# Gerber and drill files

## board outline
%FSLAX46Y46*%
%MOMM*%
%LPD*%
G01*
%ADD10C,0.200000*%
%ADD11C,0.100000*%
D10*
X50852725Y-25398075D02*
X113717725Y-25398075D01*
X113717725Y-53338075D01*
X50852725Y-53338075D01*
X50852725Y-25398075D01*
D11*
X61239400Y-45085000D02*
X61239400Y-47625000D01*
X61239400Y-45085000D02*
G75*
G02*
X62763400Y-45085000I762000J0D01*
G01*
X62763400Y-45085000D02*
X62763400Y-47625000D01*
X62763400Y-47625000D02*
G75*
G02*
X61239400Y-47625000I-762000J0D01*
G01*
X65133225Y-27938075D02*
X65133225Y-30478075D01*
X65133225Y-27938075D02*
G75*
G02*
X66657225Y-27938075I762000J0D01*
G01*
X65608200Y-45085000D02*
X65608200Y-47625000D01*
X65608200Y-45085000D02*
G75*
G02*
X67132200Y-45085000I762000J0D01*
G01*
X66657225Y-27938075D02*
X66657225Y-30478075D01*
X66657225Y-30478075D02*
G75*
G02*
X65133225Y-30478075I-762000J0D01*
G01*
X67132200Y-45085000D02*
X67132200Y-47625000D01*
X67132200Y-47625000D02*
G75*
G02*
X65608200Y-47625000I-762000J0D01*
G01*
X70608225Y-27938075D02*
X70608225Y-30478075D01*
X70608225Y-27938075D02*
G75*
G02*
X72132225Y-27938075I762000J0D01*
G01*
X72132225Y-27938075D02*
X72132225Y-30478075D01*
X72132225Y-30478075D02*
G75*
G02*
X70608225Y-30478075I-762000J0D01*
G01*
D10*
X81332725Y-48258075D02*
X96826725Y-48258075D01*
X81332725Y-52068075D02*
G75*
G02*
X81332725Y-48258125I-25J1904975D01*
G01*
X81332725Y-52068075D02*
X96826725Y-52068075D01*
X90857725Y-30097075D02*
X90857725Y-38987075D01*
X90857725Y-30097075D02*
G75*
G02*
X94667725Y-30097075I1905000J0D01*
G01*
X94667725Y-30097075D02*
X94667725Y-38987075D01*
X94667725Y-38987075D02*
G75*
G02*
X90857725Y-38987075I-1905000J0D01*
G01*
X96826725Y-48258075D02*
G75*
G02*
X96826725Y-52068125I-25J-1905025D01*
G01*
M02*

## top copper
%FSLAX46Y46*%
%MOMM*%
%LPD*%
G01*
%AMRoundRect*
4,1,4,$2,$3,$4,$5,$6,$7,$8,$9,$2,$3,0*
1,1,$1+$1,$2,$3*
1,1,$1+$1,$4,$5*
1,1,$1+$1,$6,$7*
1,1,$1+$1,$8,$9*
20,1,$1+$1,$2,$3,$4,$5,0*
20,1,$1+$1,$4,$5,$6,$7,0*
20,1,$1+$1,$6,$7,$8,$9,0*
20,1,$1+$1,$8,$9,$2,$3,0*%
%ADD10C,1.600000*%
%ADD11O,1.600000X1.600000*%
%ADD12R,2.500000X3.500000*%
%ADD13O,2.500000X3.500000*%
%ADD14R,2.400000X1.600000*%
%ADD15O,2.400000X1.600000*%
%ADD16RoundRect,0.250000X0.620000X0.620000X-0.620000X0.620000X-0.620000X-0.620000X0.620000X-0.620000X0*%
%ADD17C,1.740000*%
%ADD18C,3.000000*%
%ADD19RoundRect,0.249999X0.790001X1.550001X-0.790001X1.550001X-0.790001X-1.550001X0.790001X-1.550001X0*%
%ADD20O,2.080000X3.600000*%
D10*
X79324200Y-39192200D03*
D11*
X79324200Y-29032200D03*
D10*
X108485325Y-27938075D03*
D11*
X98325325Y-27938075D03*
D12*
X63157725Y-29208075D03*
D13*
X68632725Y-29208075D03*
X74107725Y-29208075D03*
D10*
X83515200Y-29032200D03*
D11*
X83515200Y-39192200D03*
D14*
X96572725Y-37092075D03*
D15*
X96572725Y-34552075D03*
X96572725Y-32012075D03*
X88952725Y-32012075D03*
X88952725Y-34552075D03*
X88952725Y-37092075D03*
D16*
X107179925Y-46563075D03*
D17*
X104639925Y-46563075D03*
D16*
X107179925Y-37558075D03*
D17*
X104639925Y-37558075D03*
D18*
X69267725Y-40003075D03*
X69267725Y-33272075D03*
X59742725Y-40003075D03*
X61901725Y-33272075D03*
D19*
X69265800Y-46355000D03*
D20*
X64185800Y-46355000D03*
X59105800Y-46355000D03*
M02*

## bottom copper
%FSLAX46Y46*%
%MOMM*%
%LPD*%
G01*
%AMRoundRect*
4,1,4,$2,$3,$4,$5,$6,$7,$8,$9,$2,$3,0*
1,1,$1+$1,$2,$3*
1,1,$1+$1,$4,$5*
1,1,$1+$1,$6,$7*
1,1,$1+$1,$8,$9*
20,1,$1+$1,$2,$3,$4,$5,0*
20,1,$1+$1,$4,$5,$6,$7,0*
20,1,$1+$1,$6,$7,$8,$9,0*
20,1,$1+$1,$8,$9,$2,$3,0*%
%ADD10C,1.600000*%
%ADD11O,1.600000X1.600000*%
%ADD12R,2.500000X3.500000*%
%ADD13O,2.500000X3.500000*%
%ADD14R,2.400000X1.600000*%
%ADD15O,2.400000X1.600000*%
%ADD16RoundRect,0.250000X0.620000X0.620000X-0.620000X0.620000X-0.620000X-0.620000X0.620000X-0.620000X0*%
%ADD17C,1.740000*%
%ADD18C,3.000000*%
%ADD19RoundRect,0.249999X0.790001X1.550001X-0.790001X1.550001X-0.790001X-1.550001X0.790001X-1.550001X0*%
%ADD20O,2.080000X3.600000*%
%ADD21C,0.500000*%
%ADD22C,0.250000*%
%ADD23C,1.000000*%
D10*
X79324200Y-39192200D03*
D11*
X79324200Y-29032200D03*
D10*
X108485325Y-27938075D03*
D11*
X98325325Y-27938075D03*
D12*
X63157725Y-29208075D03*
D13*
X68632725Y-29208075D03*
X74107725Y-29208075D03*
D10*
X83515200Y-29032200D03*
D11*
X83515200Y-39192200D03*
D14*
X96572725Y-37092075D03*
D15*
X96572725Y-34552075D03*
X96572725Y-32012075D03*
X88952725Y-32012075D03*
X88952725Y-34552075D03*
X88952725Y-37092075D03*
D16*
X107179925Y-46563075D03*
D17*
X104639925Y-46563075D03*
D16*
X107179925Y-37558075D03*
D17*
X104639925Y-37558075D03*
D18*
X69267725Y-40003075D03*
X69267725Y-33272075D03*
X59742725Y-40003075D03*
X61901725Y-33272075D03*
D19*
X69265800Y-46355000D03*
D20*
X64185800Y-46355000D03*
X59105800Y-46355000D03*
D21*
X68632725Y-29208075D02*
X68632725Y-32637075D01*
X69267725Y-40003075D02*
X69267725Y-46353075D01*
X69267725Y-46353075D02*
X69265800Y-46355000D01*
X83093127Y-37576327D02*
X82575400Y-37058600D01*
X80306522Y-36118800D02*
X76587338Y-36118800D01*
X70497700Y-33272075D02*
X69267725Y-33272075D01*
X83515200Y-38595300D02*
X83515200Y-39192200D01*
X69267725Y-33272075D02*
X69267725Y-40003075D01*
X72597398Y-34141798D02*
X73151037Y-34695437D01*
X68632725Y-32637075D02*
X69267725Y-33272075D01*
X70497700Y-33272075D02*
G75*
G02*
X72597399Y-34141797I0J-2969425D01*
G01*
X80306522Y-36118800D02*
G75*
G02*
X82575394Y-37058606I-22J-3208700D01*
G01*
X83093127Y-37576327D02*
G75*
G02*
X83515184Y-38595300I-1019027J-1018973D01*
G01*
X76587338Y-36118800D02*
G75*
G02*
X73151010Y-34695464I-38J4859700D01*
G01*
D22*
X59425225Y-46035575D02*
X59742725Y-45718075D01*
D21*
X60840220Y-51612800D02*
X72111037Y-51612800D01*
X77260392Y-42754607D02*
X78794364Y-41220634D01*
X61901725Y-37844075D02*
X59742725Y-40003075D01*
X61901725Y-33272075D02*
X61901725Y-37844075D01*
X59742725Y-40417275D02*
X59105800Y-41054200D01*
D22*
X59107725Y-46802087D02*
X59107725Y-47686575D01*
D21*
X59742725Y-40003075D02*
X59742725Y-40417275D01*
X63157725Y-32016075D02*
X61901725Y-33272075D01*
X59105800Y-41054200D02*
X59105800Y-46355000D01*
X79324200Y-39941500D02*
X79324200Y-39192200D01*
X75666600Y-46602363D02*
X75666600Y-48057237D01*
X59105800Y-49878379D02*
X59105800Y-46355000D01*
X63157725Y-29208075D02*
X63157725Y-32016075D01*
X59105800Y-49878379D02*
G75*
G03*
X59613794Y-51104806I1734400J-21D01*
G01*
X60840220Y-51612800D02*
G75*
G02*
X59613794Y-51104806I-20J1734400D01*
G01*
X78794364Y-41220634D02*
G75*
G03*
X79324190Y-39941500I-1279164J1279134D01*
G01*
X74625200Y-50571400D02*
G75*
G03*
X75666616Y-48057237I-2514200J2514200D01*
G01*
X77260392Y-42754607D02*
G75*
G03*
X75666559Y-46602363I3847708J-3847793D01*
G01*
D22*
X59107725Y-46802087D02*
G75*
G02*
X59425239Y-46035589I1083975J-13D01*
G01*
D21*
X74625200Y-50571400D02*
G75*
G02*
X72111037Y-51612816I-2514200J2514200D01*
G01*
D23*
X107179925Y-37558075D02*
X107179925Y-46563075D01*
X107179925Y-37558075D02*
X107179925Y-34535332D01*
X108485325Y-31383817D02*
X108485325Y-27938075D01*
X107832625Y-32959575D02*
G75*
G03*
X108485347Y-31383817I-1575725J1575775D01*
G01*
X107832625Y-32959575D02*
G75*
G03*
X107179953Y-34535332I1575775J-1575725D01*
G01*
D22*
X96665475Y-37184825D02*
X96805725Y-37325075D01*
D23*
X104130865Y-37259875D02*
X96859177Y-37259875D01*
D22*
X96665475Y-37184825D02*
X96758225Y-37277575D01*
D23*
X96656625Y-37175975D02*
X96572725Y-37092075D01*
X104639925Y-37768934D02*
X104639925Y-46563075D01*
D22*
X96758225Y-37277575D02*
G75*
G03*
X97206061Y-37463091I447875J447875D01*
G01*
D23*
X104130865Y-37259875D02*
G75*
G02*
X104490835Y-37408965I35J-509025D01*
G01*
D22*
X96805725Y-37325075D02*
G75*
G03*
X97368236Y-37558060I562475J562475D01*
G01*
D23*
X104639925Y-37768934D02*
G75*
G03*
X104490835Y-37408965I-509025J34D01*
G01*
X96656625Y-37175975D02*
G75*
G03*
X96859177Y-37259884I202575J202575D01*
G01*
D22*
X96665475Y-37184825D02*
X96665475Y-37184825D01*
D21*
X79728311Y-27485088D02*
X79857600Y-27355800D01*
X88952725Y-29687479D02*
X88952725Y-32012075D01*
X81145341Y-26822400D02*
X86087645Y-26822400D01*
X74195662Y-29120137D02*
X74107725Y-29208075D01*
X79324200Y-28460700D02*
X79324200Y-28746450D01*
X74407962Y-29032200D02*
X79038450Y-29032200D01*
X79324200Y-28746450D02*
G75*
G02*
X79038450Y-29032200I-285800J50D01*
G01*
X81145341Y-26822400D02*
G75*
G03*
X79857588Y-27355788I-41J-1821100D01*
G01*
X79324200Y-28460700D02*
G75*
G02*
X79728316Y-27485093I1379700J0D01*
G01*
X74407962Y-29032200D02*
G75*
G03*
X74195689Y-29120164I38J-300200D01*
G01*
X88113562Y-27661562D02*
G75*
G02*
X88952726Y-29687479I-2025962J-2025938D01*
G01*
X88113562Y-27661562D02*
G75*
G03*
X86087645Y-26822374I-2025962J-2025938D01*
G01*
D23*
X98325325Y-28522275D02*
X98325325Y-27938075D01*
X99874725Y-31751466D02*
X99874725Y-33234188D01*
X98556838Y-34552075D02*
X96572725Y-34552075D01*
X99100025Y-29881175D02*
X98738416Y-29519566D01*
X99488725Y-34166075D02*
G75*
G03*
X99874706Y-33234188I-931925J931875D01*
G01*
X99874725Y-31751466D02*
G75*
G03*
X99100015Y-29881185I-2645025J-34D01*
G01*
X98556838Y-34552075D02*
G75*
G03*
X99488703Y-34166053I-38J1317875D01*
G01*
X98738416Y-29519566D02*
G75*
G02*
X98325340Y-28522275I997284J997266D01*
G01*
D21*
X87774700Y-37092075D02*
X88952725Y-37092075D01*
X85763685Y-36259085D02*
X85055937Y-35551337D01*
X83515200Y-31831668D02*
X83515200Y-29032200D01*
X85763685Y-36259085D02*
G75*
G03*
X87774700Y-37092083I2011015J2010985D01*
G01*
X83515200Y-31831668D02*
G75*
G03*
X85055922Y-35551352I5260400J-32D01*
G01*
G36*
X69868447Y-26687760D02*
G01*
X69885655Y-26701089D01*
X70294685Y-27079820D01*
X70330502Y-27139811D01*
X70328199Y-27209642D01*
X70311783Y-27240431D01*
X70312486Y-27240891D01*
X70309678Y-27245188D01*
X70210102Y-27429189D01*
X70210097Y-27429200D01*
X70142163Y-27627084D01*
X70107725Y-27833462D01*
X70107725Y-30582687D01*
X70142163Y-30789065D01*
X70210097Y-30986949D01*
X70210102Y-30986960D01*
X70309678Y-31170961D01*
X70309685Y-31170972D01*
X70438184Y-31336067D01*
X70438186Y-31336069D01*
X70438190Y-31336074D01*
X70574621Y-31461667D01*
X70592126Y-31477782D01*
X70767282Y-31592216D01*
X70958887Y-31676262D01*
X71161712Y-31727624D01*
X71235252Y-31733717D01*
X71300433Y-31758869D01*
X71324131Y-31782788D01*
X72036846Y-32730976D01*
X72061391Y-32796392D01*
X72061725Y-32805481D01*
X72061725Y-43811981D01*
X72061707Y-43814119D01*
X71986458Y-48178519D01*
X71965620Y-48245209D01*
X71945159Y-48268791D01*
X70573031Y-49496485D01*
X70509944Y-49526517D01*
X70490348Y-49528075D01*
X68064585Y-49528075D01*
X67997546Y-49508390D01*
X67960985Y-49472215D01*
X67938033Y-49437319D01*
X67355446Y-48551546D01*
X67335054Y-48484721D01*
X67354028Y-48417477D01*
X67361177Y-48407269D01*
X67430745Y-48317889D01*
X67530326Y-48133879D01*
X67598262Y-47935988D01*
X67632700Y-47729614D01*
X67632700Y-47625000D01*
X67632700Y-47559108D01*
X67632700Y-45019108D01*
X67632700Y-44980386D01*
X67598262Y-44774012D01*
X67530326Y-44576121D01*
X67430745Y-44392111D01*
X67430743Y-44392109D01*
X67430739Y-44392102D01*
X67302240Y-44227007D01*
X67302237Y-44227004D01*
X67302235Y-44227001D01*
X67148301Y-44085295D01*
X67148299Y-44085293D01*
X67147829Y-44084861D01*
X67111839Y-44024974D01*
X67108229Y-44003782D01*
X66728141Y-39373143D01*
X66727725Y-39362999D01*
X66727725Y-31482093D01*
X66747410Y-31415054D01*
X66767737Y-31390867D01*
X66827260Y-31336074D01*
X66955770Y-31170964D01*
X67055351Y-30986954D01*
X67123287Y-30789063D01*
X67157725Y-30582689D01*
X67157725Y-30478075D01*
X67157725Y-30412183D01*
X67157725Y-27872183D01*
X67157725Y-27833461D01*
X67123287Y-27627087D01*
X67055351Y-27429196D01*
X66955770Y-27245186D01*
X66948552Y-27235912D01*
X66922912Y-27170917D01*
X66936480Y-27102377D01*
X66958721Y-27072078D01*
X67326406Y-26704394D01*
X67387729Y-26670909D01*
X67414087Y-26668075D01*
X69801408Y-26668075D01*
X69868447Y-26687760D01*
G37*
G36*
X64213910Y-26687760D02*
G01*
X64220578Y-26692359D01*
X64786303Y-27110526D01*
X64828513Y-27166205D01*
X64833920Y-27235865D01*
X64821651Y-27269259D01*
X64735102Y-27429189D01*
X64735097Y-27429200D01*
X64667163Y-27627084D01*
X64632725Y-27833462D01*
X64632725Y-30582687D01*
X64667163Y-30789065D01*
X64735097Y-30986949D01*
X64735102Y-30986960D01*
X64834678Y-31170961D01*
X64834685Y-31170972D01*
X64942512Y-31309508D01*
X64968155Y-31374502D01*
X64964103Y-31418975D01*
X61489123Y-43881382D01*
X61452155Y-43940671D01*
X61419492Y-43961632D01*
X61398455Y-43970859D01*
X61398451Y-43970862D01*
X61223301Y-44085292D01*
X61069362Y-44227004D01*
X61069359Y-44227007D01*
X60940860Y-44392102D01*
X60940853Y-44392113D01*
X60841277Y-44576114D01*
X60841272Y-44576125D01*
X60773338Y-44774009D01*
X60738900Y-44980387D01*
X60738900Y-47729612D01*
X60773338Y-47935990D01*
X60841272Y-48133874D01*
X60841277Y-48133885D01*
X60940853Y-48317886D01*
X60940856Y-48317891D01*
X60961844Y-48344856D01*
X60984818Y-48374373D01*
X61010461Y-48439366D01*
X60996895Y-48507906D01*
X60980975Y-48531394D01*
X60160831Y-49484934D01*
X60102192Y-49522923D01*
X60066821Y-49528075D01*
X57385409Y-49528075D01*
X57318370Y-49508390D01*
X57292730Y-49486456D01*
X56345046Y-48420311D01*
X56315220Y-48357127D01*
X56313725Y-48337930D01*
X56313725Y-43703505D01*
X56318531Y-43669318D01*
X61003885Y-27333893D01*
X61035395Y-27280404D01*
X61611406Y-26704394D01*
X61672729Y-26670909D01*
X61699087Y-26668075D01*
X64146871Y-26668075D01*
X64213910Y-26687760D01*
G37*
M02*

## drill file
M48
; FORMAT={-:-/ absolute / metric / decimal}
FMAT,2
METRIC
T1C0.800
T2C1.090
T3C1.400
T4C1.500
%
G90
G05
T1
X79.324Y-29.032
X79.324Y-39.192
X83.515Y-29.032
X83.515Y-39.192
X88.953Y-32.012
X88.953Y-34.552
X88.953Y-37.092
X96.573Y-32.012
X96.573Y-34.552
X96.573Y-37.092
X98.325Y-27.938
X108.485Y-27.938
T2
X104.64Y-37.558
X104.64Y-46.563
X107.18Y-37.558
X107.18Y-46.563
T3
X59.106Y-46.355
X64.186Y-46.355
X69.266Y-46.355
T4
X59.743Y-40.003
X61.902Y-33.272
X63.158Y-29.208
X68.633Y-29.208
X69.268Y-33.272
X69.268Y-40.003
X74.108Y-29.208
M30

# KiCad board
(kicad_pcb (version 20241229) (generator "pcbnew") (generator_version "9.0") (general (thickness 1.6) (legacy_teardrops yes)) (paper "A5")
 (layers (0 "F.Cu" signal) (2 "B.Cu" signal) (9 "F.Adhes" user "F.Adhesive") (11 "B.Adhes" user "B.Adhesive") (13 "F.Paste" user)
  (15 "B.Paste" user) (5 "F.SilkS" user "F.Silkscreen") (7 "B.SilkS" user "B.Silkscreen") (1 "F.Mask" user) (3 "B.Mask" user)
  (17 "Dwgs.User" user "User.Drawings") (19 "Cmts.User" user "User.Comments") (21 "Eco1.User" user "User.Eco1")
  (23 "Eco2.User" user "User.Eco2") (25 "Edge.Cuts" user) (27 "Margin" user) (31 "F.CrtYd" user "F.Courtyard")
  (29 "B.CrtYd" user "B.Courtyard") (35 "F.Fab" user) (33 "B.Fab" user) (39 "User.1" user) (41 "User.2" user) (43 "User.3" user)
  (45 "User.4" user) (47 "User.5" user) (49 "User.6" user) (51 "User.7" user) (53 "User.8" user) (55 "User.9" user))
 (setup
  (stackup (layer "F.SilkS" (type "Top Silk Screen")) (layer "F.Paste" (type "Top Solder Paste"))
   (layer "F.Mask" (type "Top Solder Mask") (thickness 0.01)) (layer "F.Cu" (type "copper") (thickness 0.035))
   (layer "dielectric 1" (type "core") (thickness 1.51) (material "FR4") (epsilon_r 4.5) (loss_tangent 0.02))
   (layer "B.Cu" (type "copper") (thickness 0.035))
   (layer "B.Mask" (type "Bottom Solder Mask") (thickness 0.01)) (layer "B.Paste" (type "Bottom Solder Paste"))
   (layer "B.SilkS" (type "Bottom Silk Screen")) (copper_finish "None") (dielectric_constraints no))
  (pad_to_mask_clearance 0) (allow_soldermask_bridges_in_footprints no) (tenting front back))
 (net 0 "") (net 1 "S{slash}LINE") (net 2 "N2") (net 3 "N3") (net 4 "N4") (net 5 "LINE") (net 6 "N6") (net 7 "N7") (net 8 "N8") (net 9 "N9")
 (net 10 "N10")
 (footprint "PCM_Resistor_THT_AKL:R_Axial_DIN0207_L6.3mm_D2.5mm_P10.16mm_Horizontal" (layer "F.Cu") (at 79.3242 39.1922 90)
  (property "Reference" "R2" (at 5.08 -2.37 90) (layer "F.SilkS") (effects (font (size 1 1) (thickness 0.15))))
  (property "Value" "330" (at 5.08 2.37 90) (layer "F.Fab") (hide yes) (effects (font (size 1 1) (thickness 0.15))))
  (pad "1" thru_hole circle (at 0 0 90) (size 1.6 1.6) (drill 0.8) (layers "*.Cu" "*.Mask") (remove_unused_layers no) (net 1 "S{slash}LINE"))
  (pad "2" thru_hole oval (at 10.16 0 90) (size 1.6 1.6) (drill 0.8) (layers "*.Cu" "*.Mask") (remove_unused_layers no) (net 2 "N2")))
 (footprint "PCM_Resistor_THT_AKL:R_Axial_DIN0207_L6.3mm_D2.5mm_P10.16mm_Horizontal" (layer "F.Cu") (at 108.485325 27.938075 180)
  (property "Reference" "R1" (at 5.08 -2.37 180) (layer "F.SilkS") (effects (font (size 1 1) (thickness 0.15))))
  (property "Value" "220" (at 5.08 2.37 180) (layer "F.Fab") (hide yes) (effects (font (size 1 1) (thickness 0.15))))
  (pad "1" thru_hole circle (at 0 0 180) (size 1.6 1.6) (drill 0.8) (layers "*.Cu" "*.Mask") (remove_unused_layers no) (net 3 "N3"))
  (pad "2" thru_hole oval (at 10.16 0 180) (size 1.6 1.6) (drill 0.8) (layers "*.Cu" "*.Mask") (remove_unused_layers no) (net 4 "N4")))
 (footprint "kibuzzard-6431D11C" (layer "F.Cu") (at 53.011725 39.368075 90)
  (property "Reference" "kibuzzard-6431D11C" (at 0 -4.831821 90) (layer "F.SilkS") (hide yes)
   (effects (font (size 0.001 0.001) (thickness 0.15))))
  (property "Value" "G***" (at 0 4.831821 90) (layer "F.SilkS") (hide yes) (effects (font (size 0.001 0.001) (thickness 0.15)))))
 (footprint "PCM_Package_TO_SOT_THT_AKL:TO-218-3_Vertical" (layer "F.Cu") (at 63.157725 29.208075)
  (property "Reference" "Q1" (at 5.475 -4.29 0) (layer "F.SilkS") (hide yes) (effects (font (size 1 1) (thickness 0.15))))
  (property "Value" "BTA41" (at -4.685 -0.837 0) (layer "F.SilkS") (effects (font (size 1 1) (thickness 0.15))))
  (pad "1" thru_hole rect (at 0 0) (size 2.5 3.5) (drill 1.5) (layers "*.Cu" "*.Mask") (remove_unused_layers no) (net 1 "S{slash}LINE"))
  (pad "2" thru_hole oval (at 5.475 0) (size 2.5 3.5) (drill 1.5) (layers "*.Cu" "*.Mask") (remove_unused_layers no) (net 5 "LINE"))
  (pad "3" thru_hole oval (at 10.95 0) (size 2.5 3.5) (drill 1.5) (layers "*.Cu" "*.Mask") (remove_unused_layers no) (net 2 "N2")))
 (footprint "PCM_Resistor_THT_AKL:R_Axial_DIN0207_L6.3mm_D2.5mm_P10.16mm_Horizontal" (layer "F.Cu") (at 83.5152 29.0322 -90)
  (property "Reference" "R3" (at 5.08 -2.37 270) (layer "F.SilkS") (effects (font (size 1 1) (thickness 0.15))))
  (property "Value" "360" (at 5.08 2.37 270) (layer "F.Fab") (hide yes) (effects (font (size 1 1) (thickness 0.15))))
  (pad "1" thru_hole circle (at 0 0 270) (size 1.6 1.6) (drill 0.8) (layers "*.Cu" "*.Mask") (remove_unused_layers no) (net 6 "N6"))
  (pad "2" thru_hole oval (at 10.16 0 270) (size 1.6 1.6) (drill 0.8) (layers "*.Cu" "*.Mask") (remove_unused_layers no) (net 5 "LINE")))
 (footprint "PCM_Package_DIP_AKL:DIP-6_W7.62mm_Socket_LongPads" (layer "F.Cu") (at 96.572725 37.092075 180)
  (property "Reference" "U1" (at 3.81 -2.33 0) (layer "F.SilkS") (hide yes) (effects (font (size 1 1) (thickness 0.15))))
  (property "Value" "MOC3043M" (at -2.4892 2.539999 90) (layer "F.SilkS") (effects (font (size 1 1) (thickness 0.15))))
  (pad "1" thru_hole rect (at 0 0 180) (size 2.4 1.6) (drill 0.8) (layers "*.Cu" "*.Mask") (remove_unused_layers no) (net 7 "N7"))
  (pad "2" thru_hole oval (at 0 2.54 180) (size 2.4 1.6) (drill 0.8) (layers "*.Cu" "*.Mask") (remove_unused_layers no) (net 4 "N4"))
  (pad "3" thru_hole oval (at 0 5.08 180) (size 2.4 1.6) (drill 0.8) (layers "*.Cu" "*.Mask") (remove_unused_layers no) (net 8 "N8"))
  (pad "4" thru_hole oval (at 7.62 5.08 180) (size 2.4 1.6) (drill 0.8) (layers "*.Cu" "*.Mask") (remove_unused_layers no) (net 2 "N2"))
  (pad "5" thru_hole oval (at 7.62 2.54 180) (size 2.4 1.6) (drill 0.8) (layers "*.Cu" "*.Mask") (remove_unused_layers no) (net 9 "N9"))
  (pad "6" thru_hole oval (at 7.62 0 180) (size 2.4 1.6) (drill 0.8) (layers "*.Cu" "*.Mask") (remove_unused_layers no) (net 6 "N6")))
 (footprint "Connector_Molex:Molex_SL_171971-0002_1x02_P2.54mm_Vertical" (layer "F.Cu") (at 107.179925 46.563075 180)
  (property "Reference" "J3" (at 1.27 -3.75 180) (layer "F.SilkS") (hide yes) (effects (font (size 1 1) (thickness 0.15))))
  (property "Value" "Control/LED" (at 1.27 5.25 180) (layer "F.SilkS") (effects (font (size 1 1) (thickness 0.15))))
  (pad "1" thru_hole roundrect (at 0 0 180) (size 1.74 1.74) (drill 1.09) (layers "*.Cu" "*.Mask") (remove_unused_layers no)
   (roundrect_rratio 0.143678) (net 3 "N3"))
  (pad "2" thru_hole circle (at 2.54 0 180) (size 1.74 1.74) (drill 1.09) (layers "*.Cu" "*.Mask") (remove_unused_layers no) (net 7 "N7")))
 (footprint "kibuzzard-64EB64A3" (layer "F.Cu") (at 112.041325 39.368075 -90)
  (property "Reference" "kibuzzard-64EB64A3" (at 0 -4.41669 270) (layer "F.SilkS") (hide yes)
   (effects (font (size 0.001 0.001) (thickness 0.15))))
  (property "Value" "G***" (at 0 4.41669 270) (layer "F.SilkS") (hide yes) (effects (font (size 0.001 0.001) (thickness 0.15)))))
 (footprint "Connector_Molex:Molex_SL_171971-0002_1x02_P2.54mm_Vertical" (layer "F.Cu") (at 107.179925 37.558075 180)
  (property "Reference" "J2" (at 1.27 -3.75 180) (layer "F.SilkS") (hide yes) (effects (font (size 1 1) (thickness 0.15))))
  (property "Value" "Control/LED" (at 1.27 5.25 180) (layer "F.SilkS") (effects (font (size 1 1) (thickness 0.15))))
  (pad "1" thru_hole roundrect (at 0 0 180) (size 1.74 1.74) (drill 1.09) (layers "*.Cu" "*.Mask") (remove_unused_layers no)
   (roundrect_rratio 0.143678) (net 3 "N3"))
  (pad "2" thru_hole circle (at 2.54 0 180) (size 1.74 1.74) (drill 1.09) (layers "*.Cu" "*.Mask") (remove_unused_layers no) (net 7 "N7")))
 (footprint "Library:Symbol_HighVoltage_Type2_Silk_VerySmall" (layer "F.Cu") (at 85.549125 44.676675)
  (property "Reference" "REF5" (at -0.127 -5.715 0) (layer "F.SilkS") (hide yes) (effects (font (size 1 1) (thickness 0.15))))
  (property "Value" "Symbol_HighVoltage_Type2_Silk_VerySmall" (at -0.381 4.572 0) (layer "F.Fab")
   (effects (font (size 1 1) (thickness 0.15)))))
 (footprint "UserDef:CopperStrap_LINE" (layer "F.Cu") (at 69.267725 40.003075)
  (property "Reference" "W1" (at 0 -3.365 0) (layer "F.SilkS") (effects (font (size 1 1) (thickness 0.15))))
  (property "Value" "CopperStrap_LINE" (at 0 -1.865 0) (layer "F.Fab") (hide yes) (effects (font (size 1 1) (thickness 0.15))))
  (pad "1" thru_hole circle (at 0 0) (size 3 3) (drill 1.5) (layers "*.Cu" "*.Mask") (remove_unused_layers no) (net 5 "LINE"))
  (pad "2" thru_hole circle (at 0 -6.731) (size 3 3) (drill 1.5) (layers "*.Cu" "*.Mask") (remove_unused_layers no) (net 5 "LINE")))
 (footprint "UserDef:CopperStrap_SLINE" (layer "F.Cu") (at 59.742725 40.003075)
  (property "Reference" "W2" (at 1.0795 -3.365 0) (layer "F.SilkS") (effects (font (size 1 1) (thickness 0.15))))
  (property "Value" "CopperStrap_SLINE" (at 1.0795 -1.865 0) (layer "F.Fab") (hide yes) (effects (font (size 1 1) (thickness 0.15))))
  (pad "1" thru_hole circle (at 0 0) (size 3 3) (drill 1.5) (layers "*.Cu" "*.Mask") (remove_unused_layers no) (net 1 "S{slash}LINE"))
  (pad "2" thru_hole circle (at 2.159 -6.731) (size 3 3) (drill 1.5) (layers "*.Cu" "*.Mask") (remove_unused_layers no)
   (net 1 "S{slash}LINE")))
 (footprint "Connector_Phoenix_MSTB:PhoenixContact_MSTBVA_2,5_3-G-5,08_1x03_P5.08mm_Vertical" (layer "F.Cu") (at 69.2658 46.355 180)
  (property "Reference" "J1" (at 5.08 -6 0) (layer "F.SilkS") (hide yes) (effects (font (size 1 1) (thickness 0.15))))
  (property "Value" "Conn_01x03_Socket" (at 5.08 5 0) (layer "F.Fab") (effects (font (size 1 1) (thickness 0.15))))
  (pad "1" thru_hole roundrect (at 0 0 180) (size 2.08 3.6) (drill 1.4) (layers "*.Cu" "*.Mask") (remove_unused_layers no)
   (roundrect_rratio 0.120192) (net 5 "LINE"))
  (pad "2" thru_hole oval (at 5.08 0 180) (size 2.08 3.6) (drill 1.4) (layers "*.Cu" "*.Mask") (remove_unused_layers no) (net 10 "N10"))
  (pad "3" thru_hole oval (at 10.16 0 180) (size 2.08 3.6) (drill 1.4) (layers "*.Cu" "*.Mask") (remove_unused_layers no)
   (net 1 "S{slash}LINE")))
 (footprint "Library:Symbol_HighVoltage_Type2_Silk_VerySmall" (layer "B.Cu") (at 85.549125 44.676675 180)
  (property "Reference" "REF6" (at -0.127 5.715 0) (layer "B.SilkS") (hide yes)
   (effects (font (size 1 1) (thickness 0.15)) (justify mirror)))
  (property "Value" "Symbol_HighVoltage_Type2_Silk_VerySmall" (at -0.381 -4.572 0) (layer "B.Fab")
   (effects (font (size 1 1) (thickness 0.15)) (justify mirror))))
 (gr_rect (start 50.852725 25.398075) (end 113.717725 53.338075) (stroke (width 0.2) (type default)) (fill no) (layer "Edge.Cuts"))
 (gr_line (start 61.2394 45.085) (end 61.2394 47.625) (stroke (width 0.1) (type default)) (layer "Edge.Cuts"))
 (gr_arc (start 61.2394 45.085) (mid 62.0014 44.323) (end 62.7634 45.085) (stroke (width 0.1) (type default)) (layer "Edge.Cuts"))
 (gr_line (start 62.7634 45.085) (end 62.7634 47.625) (stroke (width 0.1) (type default)) (layer "Edge.Cuts"))
 (gr_arc (start 62.7634 47.625) (mid 62.0014 48.387) (end 61.2394 47.625) (stroke (width 0.1) (type default)) (layer "Edge.Cuts"))
 (gr_line (start 65.133225 27.938075) (end 65.133225 30.478075) (stroke (width 0.1) (type default)) (layer "Edge.Cuts"))
 (gr_arc (start 65.133225 27.938075) (mid 65.895225 27.176075) (end 66.657225 27.938075) (stroke (width 0.1) (type default))
  (layer "Edge.Cuts"))
 (gr_line (start 65.6082 45.085) (end 65.6082 47.625) (stroke (width 0.1) (type default)) (layer "Edge.Cuts"))
 (gr_arc (start 65.6082 45.085) (mid 66.3702 44.323) (end 67.1322 45.085) (stroke (width 0.1) (type default)) (layer "Edge.Cuts"))
 (gr_line (start 66.657225 27.938075) (end 66.657225 30.478075) (stroke (width 0.1) (type default)) (layer "Edge.Cuts"))
 (gr_arc (start 66.657225 30.478075) (mid 65.895225 31.240075) (end 65.133225 30.478075) (stroke (width 0.1) (type default))
  (layer "Edge.Cuts"))
 (gr_line (start 67.1322 45.085) (end 67.1322 47.625) (stroke (width 0.1) (type default)) (layer "Edge.Cuts"))
 (gr_arc (start 67.1322 47.625) (mid 66.3702 48.387) (end 65.6082 47.625) (stroke (width 0.1) (type default)) (layer "Edge.Cuts"))
 (gr_line (start 70.608225 27.938075) (end 70.608225 30.478075) (stroke (width 0.1) (type default)) (layer "Edge.Cuts"))
 (gr_arc (start 70.608225 27.938075) (mid 71.370225 27.176075) (end 72.132225 27.938075) (stroke (width 0.1) (type default))
  (layer "Edge.Cuts"))
 (gr_line (start 72.132225 27.938075) (end 72.132225 30.478075) (stroke (width 0.1) (type default)) (layer "Edge.Cuts"))
 (gr_arc (start 72.132225 30.478075) (mid 71.370225 31.240075) (end 70.608225 30.478075) (stroke (width 0.1) (type default))
  (layer "Edge.Cuts"))
 (gr_line (start 81.332725 48.258075) (end 96.826725 48.258075) (stroke (width 0.2) (type default)) (layer "Edge.Cuts"))
 (gr_arc (start 81.332725 52.068075) (mid 79.427725 50.163075) (end 81.332725 48.258075) (stroke (width 0.2) (type default))
  (layer "Edge.Cuts"))
 (gr_line (start 81.332725 52.068075) (end 96.826725 52.068075) (stroke (width 0.2) (type default)) (layer "Edge.Cuts"))
 (gr_line (start 90.857725 30.097075) (end 90.857725 38.987075) (stroke (width 0.2) (type default)) (layer "Edge.Cuts"))
 (gr_arc (start 90.857725 30.097075) (mid 92.762725 28.192075) (end 94.667725 30.097075) (stroke (width 0.2) (type default))
  (layer "Edge.Cuts"))
 (gr_line (start 94.667725 30.097075) (end 94.667725 38.987075) (stroke (width 0.2) (type default)) (layer "Edge.Cuts"))
 (gr_arc (start 94.667725 38.987075) (mid 92.762725 40.892075) (end 90.857725 38.987075) (stroke (width 0.2) (type default))
  (layer "Edge.Cuts"))
 (gr_arc (start 96.826725 48.258075) (mid 98.731725 50.163075) (end 96.826725 52.068075) (stroke (width 0.2) (type default))
  (layer "Edge.Cuts"))
 (segment (start 68.632725 29.208075) (end 68.632725 32.637075) (width 0.5) (layer "B.Cu") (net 5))
 (segment (start 69.267725 40.003075) (end 69.267725 46.353075) (width 0.5) (layer "B.Cu") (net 5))
 (segment (start 69.267725 46.353075) (end 69.2658 46.355) (width 0.5) (layer "B.Cu") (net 5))
 (segment (start 83.093127 37.576327) (end 82.5754 37.0586) (width 0.5) (layer "B.Cu") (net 5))
 (segment (start 80.306522 36.1188) (end 76.587338 36.1188) (width 0.5) (layer "B.Cu") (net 5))
 (segment (start 70.4977 33.272075) (end 69.267725 33.272075) (width 0.5) (layer "B.Cu") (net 5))
 (segment (start 83.5152 38.5953) (end 83.5152 39.1922) (width 0.5) (layer "B.Cu") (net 5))
 (segment (start 69.267725 33.272075) (end 69.267725 40.003075) (width 0.5) (layer "B.Cu") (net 5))
 (segment (start 72.597398 34.141798) (end 73.151037 34.695437) (width 0.5) (layer "B.Cu") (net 5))
 (segment (start 68.632725 32.637075) (end 69.267725 33.272075) (width 0.5) (layer "B.Cu") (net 5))
 (arc (start 70.4977 33.272075) (mid 71.634048 33.498108) (end 72.597398 34.141798) (width 0.5) (layer "B.Cu") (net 5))
 (arc (start 80.306522 36.1188) (mid 81.534429 36.363046) (end 82.5754 37.0586) (width 0.5) (layer "B.Cu") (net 5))
 (arc (start 83.093127 37.576327) (mid 83.405506 38.043836) (end 83.5152 38.5953) (width 0.5) (layer "B.Cu") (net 5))
 (arc (start 76.587338 36.1188) (mid 74.727625 35.74888) (end 73.151037 34.695437) (width 0.5) (layer "B.Cu") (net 5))
 (segment (start 59.425225 46.035575) (end 59.742725 45.718075) (width 0.25) (layer "B.Cu") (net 1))
 (segment (start 60.84022 51.6128) (end 72.111037 51.6128) (width 0.5) (layer "B.Cu") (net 1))
 (segment (start 77.260392 42.754607) (end 78.794364 41.220634) (width 0.5) (layer "B.Cu") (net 1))
 (segment (start 61.901725 37.844075) (end 59.742725 40.003075) (width 0.5) (layer "B.Cu") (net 1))
 (segment (start 61.901725 33.272075) (end 61.901725 37.844075) (width 0.5) (layer "B.Cu") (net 1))
 (segment (start 59.742725 40.417275) (end 59.1058 41.0542) (width 0.5) (layer "B.Cu") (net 1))
 (segment (start 59.107725 46.802087) (end 59.107725 47.686575) (width 0.25) (layer "B.Cu") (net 1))
 (segment (start 59.742725 40.003075) (end 59.742725 40.417275) (width 0.5) (layer "B.Cu") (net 1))
 (segment (start 63.157725 32.016075) (end 61.901725 33.272075) (width 0.5) (layer "B.Cu") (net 1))
 (segment (start 59.1058 41.0542) (end 59.1058 46.355) (width 0.5) (layer "B.Cu") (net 1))
 (segment (start 79.3242 39.9415) (end 79.3242 39.1922) (width 0.5) (layer "B.Cu") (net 1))
 (segment (start 75.6666 46.602363) (end 75.6666 48.057237) (width 0.5) (layer "B.Cu") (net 1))
 (segment (start 59.1058 49.878379) (end 59.1058 46.355) (width 0.5) (layer "B.Cu") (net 1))
 (segment (start 63.157725 29.208075) (end 63.157725 32.016075) (width 0.5) (layer "B.Cu") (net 1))
 (arc (start 59.1058 49.878379) (mid 59.237824 50.542113) (end 59.6138 51.1048) (width 0.5) (layer "B.Cu") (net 1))
 (arc (start 60.84022 51.6128) (mid 60.176486 51.480775) (end 59.6138 51.1048) (width 0.5) (layer "B.Cu") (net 1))
 (arc (start 78.794364 41.220634) (mid 79.1865 40.633762) (end 79.3242 39.9415) (width 0.5) (layer "B.Cu") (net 1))
 (arc (start 74.6252 50.5714) (mid 75.395948 49.417892) (end 75.6666 48.057237) (width 0.5) (layer "B.Cu") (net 1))
 (arc (start 77.260392 42.754607) (mid 76.080813 44.519972) (end 75.6666 46.602363) (width 0.5) (layer "B.Cu") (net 1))
 (arc (start 59.107725 46.802087) (mid 59.19024 46.387253) (end 59.425225 46.035575) (width 0.25) (layer "B.Cu") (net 1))
 (arc (start 74.6252 50.5714) (mid 73.471692 51.342148) (end 72.111037 51.6128) (width 0.5) (layer "B.Cu") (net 1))
 (segment (start 107.179925 37.558075) (end 107.179925 46.563075) (width 1) (layer "B.Cu") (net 3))
 (segment (start 107.179925 37.558075) (end 107.179925 34.535332) (width 1) (layer "B.Cu") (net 3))
 (segment (start 108.485325 31.383817) (end 108.485325 27.938075) (width 1) (layer "B.Cu") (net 3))
 (arc (start 107.832625 32.959575) (mid 108.315693 32.236611) (end 108.485325 31.383817) (width 1) (layer "B.Cu") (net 3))
 (arc (start 107.832625 32.959575) (mid 107.349556 33.682538) (end 107.179925 34.535332) (width 1) (layer "B.Cu") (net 3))
 (segment (start 96.665475 37.184825) (end 96.805725 37.325075) (width 0.25) (layer "B.Cu") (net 7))
 (segment (start 104.130865 37.259875) (end 96.859177 37.259875) (width 1) (layer "B.Cu") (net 7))
 (segment (start 96.665475 37.184825) (end 96.758225 37.277575) (width 0.25) (layer "B.Cu") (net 7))
 (segment (start 96.656625 37.175975) (end 96.572725 37.092075) (width 1) (layer "B.Cu") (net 7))
 (segment (start 104.639925 37.768934) (end 104.639925 46.563075) (width 1) (layer "B.Cu") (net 7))
 (arc (start 96.758225 37.277575) (mid 96.963694 37.414865) (end 97.206061 37.463075) (width 0.25) (layer "B.Cu") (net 7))
 (arc (start 104.130865 37.259875) (mid 104.325674 37.298624) (end 104.490825 37.408975) (width 1) (layer "B.Cu") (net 7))
 (arc (start 96.805725 37.325075) (mid 97.063807 37.49752) (end 97.368236 37.558075) (width 0.25) (layer "B.Cu") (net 7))
 (arc (start 104.639925 37.768934) (mid 104.601175 37.574125) (end 104.490825 37.408975) (width 1) (layer "B.Cu") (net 7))
 (arc (start 96.656625 37.175975) (mid 96.749556 37.23807) (end 96.859177 37.259875) (width 1) (layer "B.Cu") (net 7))
 (arc (start 96.665475 37.184825) (mid 96.665475 37.184825) (end 96.665475 37.184825) (width 0.25) (layer "B.Cu") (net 7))
 (segment (start 79.728311 27.485088) (end 79.8576 27.3558) (width 0.5) (layer "B.Cu") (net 2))
 (segment (start 88.952725 29.687479) (end 88.952725 32.012075) (width 0.5) (layer "B.Cu") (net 2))
 (segment (start 81.145341 26.8224) (end 86.087645 26.8224) (width 0.5) (layer "B.Cu") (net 2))
 (segment (start 74.195662 29.120137) (end 74.107725 29.208075) (width 0.5) (layer "B.Cu") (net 2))
 (segment (start 79.3242 28.4607) (end 79.3242 28.74645) (width 0.5) (layer "B.Cu") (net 2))
 (segment (start 74.407962 29.0322) (end 79.03845 29.0322) (width 0.5) (layer "B.Cu") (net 2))
 (arc (start 79.3242 28.74645) (mid 79.240505 28.948505) (end 79.03845 29.0322) (width 0.5) (layer "B.Cu") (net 2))
 (arc (start 81.145341 26.8224) (mid 80.44842 26.961026) (end 79.8576 27.3558) (width 0.5) (layer "B.Cu") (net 2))
 (arc (start 79.3242 28.4607) (mid 79.429225 27.932702) (end 79.728311 27.485088) (width 0.5) (layer "B.Cu") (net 2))
 (arc (start 74.407962 29.0322) (mid 74.293066 29.055054) (end 74.195662 29.120137) (width 0.5) (layer "B.Cu") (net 2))
 (arc (start 88.113562 27.661562) (mid 88.734633 28.59106) (end 88.952725 29.687479) (width 0.5) (layer "B.Cu") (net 2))
 (arc (start 88.113562 27.661562) (mid 87.184063 27.040491) (end 86.087645 26.8224) (width 0.5) (layer "B.Cu") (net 2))
 (segment (start 98.325325 28.522275) (end 98.325325 27.938075) (width 1) (layer "B.Cu") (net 4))
 (segment (start 99.874725 31.751466) (end 99.874725 33.234188) (width 1) (layer "B.Cu") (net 4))
 (segment (start 98.556838 34.552075) (end 96.572725 34.552075) (width 1) (layer "B.Cu") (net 4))
 (segment (start 99.100025 29.881175) (end 98.738416 29.519566) (width 1) (layer "B.Cu") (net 4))
 (arc (start 99.488725 34.166075) (mid 99.774406 33.738521) (end 99.874725 33.234188) (width 1) (layer "B.Cu") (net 4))
 (arc (start 99.874725 31.751466) (mid 99.673387 30.739271) (end 99.100025 29.881175) (width 1) (layer "B.Cu") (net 4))
 (arc (start 98.556838 34.552075) (mid 99.061171 34.451756) (end 99.488725 34.166075) (width 1) (layer "B.Cu") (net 4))
 (arc (start 98.738416 29.519566) (mid 98.432683 29.062005) (end 98.325325 28.522275) (width 1) (layer "B.Cu") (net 4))
 (segment (start 87.7747 37.092075) (end 88.952725 37.092075) (width 0.5) (layer "B.Cu") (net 6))
 (segment (start 85.763685 36.259085) (end 85.055937 35.551337) (width 0.5) (layer "B.Cu") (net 6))
 (segment (start 83.5152 31.831668) (end 83.5152 29.0322) (width 0.5) (layer "B.Cu") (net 6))
 (arc (start 85.763685 36.259085) (mid 86.686346 36.875587) (end 87.7747 37.092075) (width 0.5) (layer "B.Cu") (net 6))
 (arc (start 83.5152 31.831668) (mid 83.915624 33.844738) (end 85.055937 35.551337) (width 0.5) (layer "B.Cu") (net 6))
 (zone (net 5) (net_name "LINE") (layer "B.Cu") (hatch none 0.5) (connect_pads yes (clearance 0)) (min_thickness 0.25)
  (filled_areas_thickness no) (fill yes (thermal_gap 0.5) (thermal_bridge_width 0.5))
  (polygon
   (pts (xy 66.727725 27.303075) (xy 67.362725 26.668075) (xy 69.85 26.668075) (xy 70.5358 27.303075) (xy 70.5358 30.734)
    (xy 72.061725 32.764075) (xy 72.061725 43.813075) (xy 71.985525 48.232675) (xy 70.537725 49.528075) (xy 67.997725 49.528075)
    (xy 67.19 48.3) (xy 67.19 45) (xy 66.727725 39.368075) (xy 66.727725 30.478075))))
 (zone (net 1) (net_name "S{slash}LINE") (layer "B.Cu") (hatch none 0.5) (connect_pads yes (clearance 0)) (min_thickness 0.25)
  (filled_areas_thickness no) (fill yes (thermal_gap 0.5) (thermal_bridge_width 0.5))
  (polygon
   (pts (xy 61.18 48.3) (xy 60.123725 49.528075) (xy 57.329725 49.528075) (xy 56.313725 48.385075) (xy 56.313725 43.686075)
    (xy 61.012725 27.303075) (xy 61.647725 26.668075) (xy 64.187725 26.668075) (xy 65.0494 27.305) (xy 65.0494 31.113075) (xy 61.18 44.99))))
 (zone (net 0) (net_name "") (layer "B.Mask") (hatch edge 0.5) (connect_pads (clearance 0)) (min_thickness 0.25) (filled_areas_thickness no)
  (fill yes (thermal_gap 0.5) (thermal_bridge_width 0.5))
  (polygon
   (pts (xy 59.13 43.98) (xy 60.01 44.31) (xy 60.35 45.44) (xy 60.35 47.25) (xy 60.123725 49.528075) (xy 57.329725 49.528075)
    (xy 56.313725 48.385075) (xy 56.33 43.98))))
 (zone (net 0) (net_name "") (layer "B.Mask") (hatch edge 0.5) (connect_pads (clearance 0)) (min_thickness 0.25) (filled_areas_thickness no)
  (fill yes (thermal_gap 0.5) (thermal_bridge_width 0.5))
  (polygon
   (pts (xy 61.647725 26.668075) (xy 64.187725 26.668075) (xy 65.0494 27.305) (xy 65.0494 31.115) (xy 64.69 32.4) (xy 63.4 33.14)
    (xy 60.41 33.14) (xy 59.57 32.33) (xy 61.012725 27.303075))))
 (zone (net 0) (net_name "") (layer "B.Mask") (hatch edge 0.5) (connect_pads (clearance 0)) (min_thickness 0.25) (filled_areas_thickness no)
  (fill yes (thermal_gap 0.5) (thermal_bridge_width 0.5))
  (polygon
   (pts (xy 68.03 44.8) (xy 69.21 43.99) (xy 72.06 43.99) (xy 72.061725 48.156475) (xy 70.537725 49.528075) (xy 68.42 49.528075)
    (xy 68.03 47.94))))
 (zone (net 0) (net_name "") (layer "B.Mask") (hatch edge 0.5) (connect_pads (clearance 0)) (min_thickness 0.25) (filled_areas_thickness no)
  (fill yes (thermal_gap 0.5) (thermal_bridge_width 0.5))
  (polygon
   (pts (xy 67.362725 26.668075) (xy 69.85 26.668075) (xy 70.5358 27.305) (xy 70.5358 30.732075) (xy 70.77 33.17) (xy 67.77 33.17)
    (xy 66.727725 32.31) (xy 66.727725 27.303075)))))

